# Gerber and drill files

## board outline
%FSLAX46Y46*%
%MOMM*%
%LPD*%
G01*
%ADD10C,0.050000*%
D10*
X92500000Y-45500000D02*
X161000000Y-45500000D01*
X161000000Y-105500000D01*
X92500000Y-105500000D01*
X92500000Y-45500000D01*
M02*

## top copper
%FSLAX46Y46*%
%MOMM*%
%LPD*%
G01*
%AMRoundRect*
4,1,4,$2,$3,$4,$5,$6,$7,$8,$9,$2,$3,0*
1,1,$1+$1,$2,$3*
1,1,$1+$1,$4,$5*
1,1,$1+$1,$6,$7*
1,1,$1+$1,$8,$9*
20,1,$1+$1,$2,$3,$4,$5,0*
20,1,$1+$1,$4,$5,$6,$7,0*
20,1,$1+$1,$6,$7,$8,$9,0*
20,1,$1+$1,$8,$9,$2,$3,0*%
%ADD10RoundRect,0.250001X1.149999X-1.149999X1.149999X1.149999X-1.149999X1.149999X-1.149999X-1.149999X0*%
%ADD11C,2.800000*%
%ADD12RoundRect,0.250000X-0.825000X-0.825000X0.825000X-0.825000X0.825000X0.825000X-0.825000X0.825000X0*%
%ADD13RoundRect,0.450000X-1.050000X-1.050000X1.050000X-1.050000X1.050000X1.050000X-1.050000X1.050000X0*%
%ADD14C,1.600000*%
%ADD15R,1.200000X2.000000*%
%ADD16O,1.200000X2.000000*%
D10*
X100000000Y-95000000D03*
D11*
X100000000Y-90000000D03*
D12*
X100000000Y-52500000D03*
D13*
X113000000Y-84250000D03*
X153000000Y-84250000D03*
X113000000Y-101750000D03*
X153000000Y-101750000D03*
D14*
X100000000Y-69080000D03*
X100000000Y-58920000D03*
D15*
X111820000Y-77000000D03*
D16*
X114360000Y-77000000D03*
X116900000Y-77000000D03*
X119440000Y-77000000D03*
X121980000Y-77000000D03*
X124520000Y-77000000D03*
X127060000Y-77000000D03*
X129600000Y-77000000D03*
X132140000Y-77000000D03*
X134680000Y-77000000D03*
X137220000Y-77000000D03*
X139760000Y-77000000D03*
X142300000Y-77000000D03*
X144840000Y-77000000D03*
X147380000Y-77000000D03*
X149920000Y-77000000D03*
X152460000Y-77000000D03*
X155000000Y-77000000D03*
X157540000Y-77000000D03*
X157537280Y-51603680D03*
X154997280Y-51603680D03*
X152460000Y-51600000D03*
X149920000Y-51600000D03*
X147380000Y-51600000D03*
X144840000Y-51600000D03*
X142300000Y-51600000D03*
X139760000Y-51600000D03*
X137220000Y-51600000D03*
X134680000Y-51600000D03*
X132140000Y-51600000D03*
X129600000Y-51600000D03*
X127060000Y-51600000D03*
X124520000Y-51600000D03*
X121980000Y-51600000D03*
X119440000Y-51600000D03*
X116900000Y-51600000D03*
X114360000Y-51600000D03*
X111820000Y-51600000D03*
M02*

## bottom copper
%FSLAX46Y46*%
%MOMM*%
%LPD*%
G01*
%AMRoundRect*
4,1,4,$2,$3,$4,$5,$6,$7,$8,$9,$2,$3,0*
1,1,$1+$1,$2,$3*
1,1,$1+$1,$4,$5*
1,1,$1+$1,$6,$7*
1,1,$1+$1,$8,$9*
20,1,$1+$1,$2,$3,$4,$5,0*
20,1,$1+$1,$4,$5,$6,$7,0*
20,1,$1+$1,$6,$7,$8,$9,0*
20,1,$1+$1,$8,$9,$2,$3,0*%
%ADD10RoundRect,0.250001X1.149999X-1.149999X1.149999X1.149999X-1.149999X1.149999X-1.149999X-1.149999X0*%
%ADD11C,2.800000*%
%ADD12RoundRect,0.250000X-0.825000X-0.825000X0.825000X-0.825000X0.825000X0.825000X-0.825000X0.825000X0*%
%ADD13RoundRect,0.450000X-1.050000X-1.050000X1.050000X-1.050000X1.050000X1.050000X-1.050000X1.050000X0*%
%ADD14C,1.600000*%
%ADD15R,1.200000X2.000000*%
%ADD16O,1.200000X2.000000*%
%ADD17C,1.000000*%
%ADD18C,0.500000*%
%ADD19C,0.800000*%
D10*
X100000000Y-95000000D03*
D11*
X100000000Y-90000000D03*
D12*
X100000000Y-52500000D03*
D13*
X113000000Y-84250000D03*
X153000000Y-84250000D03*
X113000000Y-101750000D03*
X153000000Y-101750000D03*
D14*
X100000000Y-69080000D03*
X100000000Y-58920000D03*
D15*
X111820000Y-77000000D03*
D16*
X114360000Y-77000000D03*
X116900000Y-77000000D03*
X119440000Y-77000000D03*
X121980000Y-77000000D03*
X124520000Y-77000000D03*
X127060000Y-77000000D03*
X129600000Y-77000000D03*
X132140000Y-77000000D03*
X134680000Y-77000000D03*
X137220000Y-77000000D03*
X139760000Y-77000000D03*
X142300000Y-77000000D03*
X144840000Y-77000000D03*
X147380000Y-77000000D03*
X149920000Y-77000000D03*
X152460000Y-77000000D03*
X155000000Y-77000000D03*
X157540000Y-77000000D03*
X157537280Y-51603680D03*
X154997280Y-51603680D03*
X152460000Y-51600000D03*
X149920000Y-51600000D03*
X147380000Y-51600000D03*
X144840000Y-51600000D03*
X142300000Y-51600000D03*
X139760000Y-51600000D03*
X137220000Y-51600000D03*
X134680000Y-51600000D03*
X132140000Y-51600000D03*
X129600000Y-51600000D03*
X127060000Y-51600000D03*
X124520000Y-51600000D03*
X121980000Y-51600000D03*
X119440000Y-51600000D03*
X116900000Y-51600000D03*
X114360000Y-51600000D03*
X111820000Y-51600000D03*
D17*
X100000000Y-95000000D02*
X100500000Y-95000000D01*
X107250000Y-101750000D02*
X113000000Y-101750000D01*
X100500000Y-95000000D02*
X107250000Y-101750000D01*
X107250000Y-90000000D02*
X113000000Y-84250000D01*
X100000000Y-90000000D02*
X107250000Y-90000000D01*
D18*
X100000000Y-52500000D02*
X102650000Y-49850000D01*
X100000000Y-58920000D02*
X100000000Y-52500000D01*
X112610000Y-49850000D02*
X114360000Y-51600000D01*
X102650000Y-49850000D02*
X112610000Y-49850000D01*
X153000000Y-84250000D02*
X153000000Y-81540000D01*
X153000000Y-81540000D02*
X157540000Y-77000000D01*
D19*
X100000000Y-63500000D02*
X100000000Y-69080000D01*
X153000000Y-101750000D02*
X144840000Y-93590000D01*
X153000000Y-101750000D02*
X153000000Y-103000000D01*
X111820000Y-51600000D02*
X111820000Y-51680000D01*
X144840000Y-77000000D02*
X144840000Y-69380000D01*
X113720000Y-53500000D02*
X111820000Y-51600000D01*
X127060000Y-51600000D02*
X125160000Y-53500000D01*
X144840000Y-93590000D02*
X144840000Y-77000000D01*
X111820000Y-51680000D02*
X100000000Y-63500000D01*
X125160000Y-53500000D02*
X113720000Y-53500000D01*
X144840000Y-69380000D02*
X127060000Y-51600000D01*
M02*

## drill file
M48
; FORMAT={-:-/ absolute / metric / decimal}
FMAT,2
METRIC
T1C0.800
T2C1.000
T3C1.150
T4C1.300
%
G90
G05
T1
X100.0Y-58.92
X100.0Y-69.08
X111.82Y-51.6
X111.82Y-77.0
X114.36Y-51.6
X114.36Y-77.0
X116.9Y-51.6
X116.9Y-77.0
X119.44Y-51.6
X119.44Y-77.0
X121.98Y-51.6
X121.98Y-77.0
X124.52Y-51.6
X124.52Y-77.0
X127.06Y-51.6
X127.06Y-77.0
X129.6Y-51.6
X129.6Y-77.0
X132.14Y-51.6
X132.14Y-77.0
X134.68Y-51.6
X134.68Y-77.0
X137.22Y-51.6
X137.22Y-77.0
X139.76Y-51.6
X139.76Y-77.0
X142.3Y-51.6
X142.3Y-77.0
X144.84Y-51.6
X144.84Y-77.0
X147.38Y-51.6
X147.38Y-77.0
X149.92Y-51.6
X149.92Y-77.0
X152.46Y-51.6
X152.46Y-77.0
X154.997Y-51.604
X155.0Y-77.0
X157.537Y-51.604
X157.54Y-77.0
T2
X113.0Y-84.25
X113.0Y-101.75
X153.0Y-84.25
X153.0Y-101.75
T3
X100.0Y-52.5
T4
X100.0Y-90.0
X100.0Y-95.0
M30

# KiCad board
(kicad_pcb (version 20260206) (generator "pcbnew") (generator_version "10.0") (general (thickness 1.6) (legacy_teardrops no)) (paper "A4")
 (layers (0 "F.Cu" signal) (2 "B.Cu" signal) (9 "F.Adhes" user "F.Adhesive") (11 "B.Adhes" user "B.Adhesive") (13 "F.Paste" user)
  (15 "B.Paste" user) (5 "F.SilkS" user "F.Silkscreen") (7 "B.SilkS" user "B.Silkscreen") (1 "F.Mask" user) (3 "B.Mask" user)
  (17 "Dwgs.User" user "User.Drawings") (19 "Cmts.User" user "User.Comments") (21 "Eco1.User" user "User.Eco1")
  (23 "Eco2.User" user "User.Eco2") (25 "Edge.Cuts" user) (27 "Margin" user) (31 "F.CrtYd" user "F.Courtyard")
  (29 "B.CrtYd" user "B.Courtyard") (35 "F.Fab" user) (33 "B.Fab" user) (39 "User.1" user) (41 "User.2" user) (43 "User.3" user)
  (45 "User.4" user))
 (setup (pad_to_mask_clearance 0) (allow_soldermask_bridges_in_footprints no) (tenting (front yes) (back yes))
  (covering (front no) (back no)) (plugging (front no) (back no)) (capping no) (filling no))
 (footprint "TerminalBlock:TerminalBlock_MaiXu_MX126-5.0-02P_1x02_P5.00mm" (layer "F.Cu") (at 100 95 90)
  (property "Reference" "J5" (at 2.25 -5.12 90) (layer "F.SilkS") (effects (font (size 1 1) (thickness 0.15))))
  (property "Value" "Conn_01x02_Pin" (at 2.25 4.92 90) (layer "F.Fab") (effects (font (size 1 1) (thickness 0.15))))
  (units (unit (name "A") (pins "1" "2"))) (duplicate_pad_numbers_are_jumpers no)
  (pad "1" thru_hole roundrect (at 0 0 90) (size 2.8 2.8) (drill 1.3) (layers "*.Cu" "*.Mask") (remove_unused_layers no)
   (roundrect_rratio 0.089286) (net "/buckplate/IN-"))
  (pad "2" thru_hole circle (at 5 0 90) (size 2.8 2.8) (drill 1.3) (layers "*.Cu" "*.Mask") (remove_unused_layers no) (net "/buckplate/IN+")))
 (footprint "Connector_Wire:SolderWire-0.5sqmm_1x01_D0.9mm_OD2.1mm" (layer "F.Cu") (at 100 52.5)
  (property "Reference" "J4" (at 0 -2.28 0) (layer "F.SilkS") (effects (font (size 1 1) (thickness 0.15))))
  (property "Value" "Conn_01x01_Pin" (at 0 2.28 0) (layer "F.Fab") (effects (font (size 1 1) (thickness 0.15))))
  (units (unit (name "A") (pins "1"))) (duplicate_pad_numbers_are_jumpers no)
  (pad "1" thru_hole roundrect (at 0 0) (size 2.15 2.15) (drill 1.15) (layers "*.Cu" "*.Mask") (remove_unused_layers no)
   (roundrect_rratio 0.116279) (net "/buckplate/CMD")))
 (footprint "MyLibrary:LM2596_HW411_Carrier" (layer "F.Cu") (at 113 101.75)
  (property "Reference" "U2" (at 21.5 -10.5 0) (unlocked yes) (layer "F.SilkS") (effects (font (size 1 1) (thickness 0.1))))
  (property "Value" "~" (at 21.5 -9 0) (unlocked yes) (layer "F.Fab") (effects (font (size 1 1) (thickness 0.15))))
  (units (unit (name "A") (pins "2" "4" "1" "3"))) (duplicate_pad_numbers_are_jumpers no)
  (pad "1" thru_hole roundrect (at 0 -17.5) (size 3 3) (drill 1) (layers "*.Cu" "*.Mask") (remove_unused_layers no) (roundrect_rratio 0.15)
   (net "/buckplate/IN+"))
  (pad "2" thru_hole roundrect (at 40 -17.5) (size 3 3) (drill 1) (layers "*.Cu" "*.Mask") (remove_unused_layers no) (roundrect_rratio 0.15)
   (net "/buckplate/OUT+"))
  (pad "3" thru_hole roundrect (at 0 0) (size 3 3) (drill 1) (layers "*.Cu" "*.Mask") (remove_unused_layers no) (roundrect_rratio 0.15)
   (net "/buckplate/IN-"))
  (pad "4" thru_hole roundrect (at 40 0) (size 3 3) (drill 1) (layers "*.Cu" "*.Mask") (remove_unused_layers no) (roundrect_rratio 0.15)
   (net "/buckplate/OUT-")))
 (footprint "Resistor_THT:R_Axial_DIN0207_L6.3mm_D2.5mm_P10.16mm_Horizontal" (layer "F.Cu") (at 100 69.08 90)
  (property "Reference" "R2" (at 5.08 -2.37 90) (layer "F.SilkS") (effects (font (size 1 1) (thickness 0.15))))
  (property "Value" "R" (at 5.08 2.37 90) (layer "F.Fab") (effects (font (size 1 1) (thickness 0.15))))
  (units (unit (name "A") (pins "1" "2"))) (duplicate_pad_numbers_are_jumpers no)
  (pad "1" thru_hole circle (at 0 0 90) (size 1.6 1.6) (drill 0.8) (layers "*.Cu" "*.Mask") (remove_unused_layers no)
   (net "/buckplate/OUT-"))
  (pad "2" thru_hole circle (at 10.16 0 90) (size 1.6 1.6) (drill 0.8) (layers "*.Cu" "*.Mask") (remove_unused_layers no)
   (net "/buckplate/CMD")))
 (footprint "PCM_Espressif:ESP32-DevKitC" (layer "F.Cu") (at 111.82 77 90)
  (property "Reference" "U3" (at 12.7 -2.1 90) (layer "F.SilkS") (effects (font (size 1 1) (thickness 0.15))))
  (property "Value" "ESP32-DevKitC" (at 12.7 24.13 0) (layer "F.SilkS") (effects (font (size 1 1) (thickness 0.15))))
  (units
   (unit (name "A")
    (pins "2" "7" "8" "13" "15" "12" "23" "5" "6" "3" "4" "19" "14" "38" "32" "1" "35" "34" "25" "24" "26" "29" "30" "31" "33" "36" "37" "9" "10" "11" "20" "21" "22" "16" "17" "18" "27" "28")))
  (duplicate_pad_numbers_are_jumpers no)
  (pad "1" thru_hole rect (at 0 0) (size 1.2 2) (drill 0.8) (layers "*.Cu" "*.Mask") (remove_unused_layers no)
   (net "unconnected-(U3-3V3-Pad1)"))
  (pad "2" thru_hole oval (at 0 2.54) (size 1.2 2) (drill 0.8) (layers "*.Cu" "*.Mask") (remove_unused_layers no)
   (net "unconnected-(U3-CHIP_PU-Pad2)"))
  (pad "3" thru_hole oval (at 0 5.08) (size 1.2 2) (drill 0.8) (layers "*.Cu" "*.Mask") (remove_unused_layers no)
   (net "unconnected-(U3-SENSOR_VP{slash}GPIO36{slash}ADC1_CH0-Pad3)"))
  (pad "4" thru_hole oval (at 0 7.62) (size 1.2 2) (drill 0.8) (layers "*.Cu" "*.Mask") (remove_unused_layers no)
   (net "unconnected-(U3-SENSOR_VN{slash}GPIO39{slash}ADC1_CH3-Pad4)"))
  (pad "5" thru_hole oval (at 0 10.16) (size 1.2 2) (drill 0.8) (layers "*.Cu" "*.Mask") (remove_unused_layers no)
   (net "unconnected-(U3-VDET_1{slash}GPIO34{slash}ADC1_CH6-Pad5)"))
  (pad "6" thru_hole oval (at 0 12.7) (size 1.2 2) (drill 0.8) (layers "*.Cu" "*.Mask") (remove_unused_layers no)
   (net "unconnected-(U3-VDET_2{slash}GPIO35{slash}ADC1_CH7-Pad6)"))
  (pad "7" thru_hole oval (at 0 15.24) (size 1.2 2) (drill 0.8) (layers "*.Cu" "*.Mask") (remove_unused_layers no)
   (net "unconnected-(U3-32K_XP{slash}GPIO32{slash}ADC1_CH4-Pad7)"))
  (pad "8" thru_hole oval (at 0 17.78) (size 1.2 2) (drill 0.8) (layers "*.Cu" "*.Mask") (remove_unused_layers no)
   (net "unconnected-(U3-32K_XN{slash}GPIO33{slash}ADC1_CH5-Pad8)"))
  (pad "9" thru_hole oval (at 0 20.32) (size 1.2 2) (drill 0.8) (layers "*.Cu" "*.Mask") (remove_unused_layers no)
   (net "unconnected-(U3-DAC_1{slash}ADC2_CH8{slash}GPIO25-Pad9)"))
  (pad "10" thru_hole oval (at 0 22.86) (size 1.2 2) (drill 0.8) (layers "*.Cu" "*.Mask") (remove_unused_layers no)
   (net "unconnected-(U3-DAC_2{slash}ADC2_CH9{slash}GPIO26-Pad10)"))
  (pad "11" thru_hole oval (at 0 25.4) (size 1.2 2) (drill 0.8) (layers "*.Cu" "*.Mask") (remove_unused_layers no)
   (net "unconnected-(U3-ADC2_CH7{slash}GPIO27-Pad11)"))
  (pad "12" thru_hole oval (at 0 27.94) (size 1.2 2) (drill 0.8) (layers "*.Cu" "*.Mask") (remove_unused_layers no)
   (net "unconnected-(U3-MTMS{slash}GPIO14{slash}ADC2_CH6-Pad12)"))
  (pad "13" thru_hole oval (at 0 30.48) (size 1.2 2) (drill 0.8) (layers "*.Cu" "*.Mask") (remove_unused_layers no)
   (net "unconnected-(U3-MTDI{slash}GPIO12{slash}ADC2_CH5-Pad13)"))
  (pad "14" thru_hole oval (at 0 33.02) (size 1.2 2) (drill 0.8) (layers "*.Cu" "*.Mask") (remove_unused_layers no) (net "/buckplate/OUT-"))
  (pad "15" thru_hole oval (at 0 35.56) (size 1.2 2) (drill 0.8) (layers "*.Cu" "*.Mask") (remove_unused_layers no)
   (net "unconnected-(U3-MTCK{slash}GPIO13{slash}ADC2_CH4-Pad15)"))
  (pad "16" thru_hole oval (at 0 38.1) (size 1.2 2) (drill 0.8) (layers "*.Cu" "*.Mask") (remove_unused_layers no)
   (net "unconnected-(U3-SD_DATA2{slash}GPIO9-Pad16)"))
  (pad "17" thru_hole oval (at 0 40.64) (size 1.2 2) (drill 0.8) (layers "*.Cu" "*.Mask") (remove_unused_layers no)
   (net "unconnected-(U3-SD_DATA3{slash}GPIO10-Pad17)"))
  (pad "18" thru_hole oval (at 0 43.18) (size 1.2 2) (drill 0.8) (layers "*.Cu" "*.Mask") (remove_unused_layers no)
   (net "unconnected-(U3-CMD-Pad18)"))
  (pad "19" thru_hole oval (at 0 45.72) (size 1.2 2) (drill 0.8) (layers "*.Cu" "*.Mask") (remove_unused_layers no) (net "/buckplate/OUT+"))
  (pad "20" thru_hole oval (at 25.39632 45.71728) (size 1.2 2) (drill 0.8) (layers "*.Cu" "*.Mask") (remove_unused_layers no)
   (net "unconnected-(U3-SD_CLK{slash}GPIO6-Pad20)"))
  (pad "21" thru_hole oval (at 25.39632 43.17728) (size 1.2 2) (drill 0.8) (layers "*.Cu" "*.Mask") (remove_unused_layers no)
   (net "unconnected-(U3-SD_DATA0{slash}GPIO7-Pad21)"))
  (pad "22" thru_hole oval (at 25.4 40.64) (size 1.2 2) (drill 0.8) (layers "*.Cu" "*.Mask") (remove_unused_layers no)
   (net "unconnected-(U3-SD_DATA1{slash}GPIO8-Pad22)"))
  (pad "23" thru_hole oval (at 25.4 38.1) (size 1.2 2) (drill 0.8) (layers "*.Cu" "*.Mask") (remove_unused_layers no)
   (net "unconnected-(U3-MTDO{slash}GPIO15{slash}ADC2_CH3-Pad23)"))
  (pad "24" thru_hole oval (at 25.4 35.56) (size 1.2 2) (drill 0.8) (layers "*.Cu" "*.Mask") (remove_unused_layers no)
   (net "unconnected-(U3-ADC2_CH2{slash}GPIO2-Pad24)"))
  (pad "25" thru_hole oval (at 25.4 33.02) (size 1.2 2) (drill 0.8) (layers "*.Cu" "*.Mask") (remove_unused_layers no)
   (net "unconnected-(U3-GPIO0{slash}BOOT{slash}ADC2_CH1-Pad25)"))
  (pad "26" thru_hole oval (at 25.4 30.48) (size 1.2 2) (drill 0.8) (layers "*.Cu" "*.Mask") (remove_unused_layers no)
   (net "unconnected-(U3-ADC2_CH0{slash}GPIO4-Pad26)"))
  (pad "27" thru_hole oval (at 25.4 27.94) (size 1.2 2) (drill 0.8) (layers "*.Cu" "*.Mask") (remove_unused_layers no)
   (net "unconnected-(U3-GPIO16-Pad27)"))
  (pad "28" thru_hole oval (at 25.4 25.4) (size 1.2 2) (drill 0.8) (layers "*.Cu" "*.Mask") (remove_unused_layers no)
   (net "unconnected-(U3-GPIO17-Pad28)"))
  (pad "29" thru_hole oval (at 25.4 22.86) (size 1.2 2) (drill 0.8) (layers "*.Cu" "*.Mask") (remove_unused_layers no)
   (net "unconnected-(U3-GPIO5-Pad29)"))
  (pad "30" thru_hole oval (at 25.4 20.32) (size 1.2 2) (drill 0.8) (layers "*.Cu" "*.Mask") (remove_unused_layers no)
   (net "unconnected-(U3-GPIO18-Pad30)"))
  (pad "31" thru_hole oval (at 25.4 17.78) (size 1.2 2) (drill 0.8) (layers "*.Cu" "*.Mask") (remove_unused_layers no)
   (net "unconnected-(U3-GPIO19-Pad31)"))
  (pad "32" thru_hole oval (at 25.4 15.24) (size 1.2 2) (drill 0.8) (layers "*.Cu" "*.Mask") (remove_unused_layers no)
   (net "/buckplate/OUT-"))
  (pad "33" thru_hole oval (at 25.4 12.7) (size 1.2 2) (drill 0.8) (layers "*.Cu" "*.Mask") (remove_unused_layers no)
   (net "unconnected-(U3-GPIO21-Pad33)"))
  (pad "34" thru_hole oval (at 25.4 10.16) (size 1.2 2) (drill 0.8) (layers "*.Cu" "*.Mask") (remove_unused_layers no)
   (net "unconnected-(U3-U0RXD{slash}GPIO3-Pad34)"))
  (pad "35" thru_hole oval (at 25.4 7.62) (size 1.2 2) (drill 0.8) (layers "*.Cu" "*.Mask") (remove_unused_layers no)
   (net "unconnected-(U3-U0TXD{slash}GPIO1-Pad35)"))
  (pad "36" thru_hole oval (at 25.4 5.08) (size 1.2 2) (drill 0.8) (layers "*.Cu" "*.Mask") (remove_unused_layers no)
   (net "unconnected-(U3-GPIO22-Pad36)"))
  (pad "37" thru_hole oval (at 25.4 2.54) (size 1.2 2) (drill 0.8) (layers "*.Cu" "*.Mask") (remove_unused_layers no) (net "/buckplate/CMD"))
  (pad "38" thru_hole oval (at 25.4 0) (size 1.2 2) (drill 0.8) (layers "*.Cu" "*.Mask") (remove_unused_layers no) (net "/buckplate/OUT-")))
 (gr_rect (start 92.5 45.5) (end 161 105.5) (stroke (width 0.05) (type default)) (fill no) (layer "Edge.Cuts"))
 (segment (start 100 95) (end 100.5 95) (width 1) (layer "B.Cu") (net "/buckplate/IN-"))
 (segment (start 107.25 101.75) (end 113 101.75) (width 1) (layer "B.Cu") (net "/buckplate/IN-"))
 (segment (start 100.5 95) (end 107.25 101.75) (width 1) (layer "B.Cu") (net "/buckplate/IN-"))
 (segment (start 107.25 90) (end 113 84.25) (width 1) (layer "B.Cu") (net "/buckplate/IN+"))
 (segment (start 100 90) (end 107.25 90) (width 1) (layer "B.Cu") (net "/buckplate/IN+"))
 (segment (start 100 52.5) (end 102.65 49.85) (width 0.5) (layer "B.Cu") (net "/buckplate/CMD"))
 (segment (start 100 58.92) (end 100 52.5) (width 0.5) (layer "B.Cu") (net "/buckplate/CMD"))
 (segment (start 112.61 49.85) (end 114.36 51.6) (width 0.5) (layer "B.Cu") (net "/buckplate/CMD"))
 (segment (start 102.65 49.85) (end 112.61 49.85) (width 0.5) (layer "B.Cu") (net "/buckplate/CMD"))
 (segment (start 153 84.25) (end 153 81.54) (width 0.5) (layer "B.Cu") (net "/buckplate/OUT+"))
 (segment (start 153 81.54) (end 157.54 77) (width 0.5) (layer "B.Cu") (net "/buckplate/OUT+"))
 (segment (start 100 63.5) (end 100 69.08) (width 0.8) (layer "B.Cu") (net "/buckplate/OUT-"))
 (segment (start 153 101.75) (end 144.84 93.59) (width 0.8) (layer "B.Cu") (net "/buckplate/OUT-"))
 (segment (start 153 101.75) (end 153 103) (width 0.8) (layer "B.Cu") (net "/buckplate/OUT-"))
 (segment (start 111.82 51.6) (end 111.82 51.68) (width 0.8) (layer "B.Cu") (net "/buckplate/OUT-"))
 (segment (start 144.84 77) (end 144.84 69.38) (width 0.8) (layer "B.Cu") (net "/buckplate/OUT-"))
 (segment (start 113.72 53.5) (end 111.82 51.6) (width 0.8) (layer "B.Cu") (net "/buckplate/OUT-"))
 (segment (start 127.06 51.6) (end 125.16 53.5) (width 0.8) (layer "B.Cu") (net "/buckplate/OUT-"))
 (segment (start 144.84 93.59) (end 144.84 77) (width 0.8) (layer "B.Cu") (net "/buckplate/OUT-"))
 (segment (start 111.82 51.68) (end 100 63.5) (width 0.8) (layer "B.Cu") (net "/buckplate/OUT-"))
 (segment (start 125.16 53.5) (end 113.72 53.5) (width 0.8) (layer "B.Cu") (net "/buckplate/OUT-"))
 (segment (start 144.84 69.38) (end 127.06 51.6) (width 0.8) (layer "B.Cu") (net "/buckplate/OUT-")))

